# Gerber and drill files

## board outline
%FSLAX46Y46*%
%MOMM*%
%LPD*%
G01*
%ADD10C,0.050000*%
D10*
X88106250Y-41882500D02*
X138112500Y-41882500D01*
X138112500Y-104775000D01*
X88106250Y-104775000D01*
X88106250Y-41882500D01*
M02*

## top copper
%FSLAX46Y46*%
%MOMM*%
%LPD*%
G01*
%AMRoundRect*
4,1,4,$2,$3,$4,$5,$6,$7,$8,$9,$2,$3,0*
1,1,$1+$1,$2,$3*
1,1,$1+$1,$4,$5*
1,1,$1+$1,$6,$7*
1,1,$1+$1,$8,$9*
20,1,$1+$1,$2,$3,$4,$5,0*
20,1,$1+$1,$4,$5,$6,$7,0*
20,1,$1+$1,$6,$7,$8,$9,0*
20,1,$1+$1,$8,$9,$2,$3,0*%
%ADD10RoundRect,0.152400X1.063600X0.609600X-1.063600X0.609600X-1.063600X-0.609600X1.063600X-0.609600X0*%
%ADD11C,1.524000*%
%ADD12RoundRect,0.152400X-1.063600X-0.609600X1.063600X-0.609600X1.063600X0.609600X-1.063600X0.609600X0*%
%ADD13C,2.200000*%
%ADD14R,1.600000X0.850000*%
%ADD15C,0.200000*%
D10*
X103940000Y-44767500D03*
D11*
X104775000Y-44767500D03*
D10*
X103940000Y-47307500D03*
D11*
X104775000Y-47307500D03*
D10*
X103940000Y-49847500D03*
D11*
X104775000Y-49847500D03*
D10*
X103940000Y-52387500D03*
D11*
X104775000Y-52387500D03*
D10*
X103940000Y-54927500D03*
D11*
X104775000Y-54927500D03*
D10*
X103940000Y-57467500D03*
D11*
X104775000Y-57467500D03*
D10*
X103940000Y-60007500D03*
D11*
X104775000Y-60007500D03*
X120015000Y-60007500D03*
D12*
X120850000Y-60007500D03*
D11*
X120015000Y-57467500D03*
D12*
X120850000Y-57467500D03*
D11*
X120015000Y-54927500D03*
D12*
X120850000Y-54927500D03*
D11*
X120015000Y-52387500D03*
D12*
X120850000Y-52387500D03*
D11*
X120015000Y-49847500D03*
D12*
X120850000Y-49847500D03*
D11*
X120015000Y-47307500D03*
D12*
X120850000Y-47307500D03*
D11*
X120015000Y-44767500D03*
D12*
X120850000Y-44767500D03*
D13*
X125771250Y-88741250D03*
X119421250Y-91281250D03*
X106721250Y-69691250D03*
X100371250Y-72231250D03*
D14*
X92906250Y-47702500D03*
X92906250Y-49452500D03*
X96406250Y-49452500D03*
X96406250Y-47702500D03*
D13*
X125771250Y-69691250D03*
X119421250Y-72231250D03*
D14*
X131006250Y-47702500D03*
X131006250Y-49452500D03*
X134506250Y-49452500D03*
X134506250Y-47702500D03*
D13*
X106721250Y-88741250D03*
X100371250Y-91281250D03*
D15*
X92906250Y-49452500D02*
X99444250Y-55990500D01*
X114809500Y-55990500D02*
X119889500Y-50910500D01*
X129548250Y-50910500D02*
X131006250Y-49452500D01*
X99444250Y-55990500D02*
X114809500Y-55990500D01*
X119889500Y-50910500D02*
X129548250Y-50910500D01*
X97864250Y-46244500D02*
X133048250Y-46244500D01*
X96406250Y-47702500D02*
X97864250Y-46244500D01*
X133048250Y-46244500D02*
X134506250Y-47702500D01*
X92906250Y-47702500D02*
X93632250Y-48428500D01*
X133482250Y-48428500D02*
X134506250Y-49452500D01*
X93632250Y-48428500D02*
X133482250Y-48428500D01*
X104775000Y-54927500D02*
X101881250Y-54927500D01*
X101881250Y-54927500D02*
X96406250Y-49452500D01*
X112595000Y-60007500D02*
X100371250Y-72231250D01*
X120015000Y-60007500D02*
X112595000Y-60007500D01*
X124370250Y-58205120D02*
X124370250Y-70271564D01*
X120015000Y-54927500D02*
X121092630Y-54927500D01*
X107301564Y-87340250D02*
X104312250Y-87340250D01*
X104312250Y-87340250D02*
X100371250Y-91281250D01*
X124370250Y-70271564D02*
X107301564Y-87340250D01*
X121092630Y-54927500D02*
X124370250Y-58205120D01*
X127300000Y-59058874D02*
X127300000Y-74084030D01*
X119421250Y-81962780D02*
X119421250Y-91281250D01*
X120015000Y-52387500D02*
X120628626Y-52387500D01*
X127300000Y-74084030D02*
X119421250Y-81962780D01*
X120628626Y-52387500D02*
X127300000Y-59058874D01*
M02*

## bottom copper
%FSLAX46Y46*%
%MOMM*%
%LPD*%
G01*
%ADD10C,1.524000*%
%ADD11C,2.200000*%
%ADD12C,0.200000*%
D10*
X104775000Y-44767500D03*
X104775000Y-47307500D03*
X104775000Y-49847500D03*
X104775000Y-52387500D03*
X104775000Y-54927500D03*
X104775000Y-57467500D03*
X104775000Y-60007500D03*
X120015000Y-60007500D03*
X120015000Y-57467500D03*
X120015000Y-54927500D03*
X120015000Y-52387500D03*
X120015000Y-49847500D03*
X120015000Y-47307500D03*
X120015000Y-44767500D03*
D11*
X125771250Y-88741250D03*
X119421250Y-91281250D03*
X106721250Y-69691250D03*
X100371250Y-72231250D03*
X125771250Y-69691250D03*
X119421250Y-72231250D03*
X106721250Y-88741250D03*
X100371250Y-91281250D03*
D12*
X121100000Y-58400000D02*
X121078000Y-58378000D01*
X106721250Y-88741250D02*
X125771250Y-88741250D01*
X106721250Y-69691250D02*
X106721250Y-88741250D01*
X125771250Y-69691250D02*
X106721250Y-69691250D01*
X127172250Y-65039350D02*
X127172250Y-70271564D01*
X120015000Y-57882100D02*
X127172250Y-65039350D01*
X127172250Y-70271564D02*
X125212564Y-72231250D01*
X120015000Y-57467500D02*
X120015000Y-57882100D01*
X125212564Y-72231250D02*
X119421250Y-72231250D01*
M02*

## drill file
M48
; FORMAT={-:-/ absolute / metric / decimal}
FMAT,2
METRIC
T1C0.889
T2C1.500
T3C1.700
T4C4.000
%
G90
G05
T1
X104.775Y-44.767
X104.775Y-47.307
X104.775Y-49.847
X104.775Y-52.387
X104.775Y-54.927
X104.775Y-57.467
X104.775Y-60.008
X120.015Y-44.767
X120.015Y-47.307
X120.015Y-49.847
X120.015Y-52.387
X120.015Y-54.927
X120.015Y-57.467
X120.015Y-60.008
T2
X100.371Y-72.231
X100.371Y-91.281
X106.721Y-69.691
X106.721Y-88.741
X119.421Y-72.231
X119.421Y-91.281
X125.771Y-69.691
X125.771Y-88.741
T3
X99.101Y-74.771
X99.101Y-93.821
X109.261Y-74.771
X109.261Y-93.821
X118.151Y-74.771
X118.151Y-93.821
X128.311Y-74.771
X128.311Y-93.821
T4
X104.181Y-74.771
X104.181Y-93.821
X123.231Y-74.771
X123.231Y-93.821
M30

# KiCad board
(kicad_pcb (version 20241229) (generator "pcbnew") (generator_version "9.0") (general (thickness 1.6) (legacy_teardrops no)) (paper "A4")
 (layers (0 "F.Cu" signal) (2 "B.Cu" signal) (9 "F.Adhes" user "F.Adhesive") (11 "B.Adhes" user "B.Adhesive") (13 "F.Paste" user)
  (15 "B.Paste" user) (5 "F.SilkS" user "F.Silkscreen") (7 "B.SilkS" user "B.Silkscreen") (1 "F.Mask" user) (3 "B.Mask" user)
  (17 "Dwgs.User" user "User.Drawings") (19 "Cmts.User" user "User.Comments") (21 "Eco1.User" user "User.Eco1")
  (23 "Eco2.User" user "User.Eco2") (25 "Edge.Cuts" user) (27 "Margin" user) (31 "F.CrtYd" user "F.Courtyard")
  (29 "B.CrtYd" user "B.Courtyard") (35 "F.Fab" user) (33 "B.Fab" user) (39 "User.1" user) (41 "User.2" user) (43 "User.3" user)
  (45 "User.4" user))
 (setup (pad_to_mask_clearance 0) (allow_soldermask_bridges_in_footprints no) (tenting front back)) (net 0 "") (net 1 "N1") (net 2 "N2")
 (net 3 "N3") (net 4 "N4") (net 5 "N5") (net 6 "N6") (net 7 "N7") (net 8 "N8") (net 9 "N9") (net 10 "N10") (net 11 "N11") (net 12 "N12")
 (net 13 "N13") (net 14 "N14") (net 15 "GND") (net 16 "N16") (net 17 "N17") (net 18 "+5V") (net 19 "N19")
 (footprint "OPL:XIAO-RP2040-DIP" (layer "F.Cu") (at 112.395 52.3875)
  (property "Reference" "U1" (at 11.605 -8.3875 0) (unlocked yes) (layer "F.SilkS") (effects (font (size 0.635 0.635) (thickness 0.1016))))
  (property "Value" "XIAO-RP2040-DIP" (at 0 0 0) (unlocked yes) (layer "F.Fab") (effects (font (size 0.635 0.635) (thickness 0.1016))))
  (pad "1" smd roundrect (at -8.455 -7.62 180) (size 2.432 1.524) (layers "F.Cu" "F.Mask") (roundrect_rratio 0.1) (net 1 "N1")
   (thermal_bridge_angle 45))
  (pad "1" thru_hole circle (at -7.62 -7.62 180) (size 1.524 1.524) (drill 0.889) (layers "*.Cu" "*.Mask") (remove_unused_layers no)
   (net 1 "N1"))
  (pad "2" smd roundrect (at -8.455 -5.08 180) (size 2.432 1.524) (layers "F.Cu" "F.Mask") (roundrect_rratio 0.1) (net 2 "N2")
   (thermal_bridge_angle 45))
  (pad "2" thru_hole circle (at -7.62 -5.08 180) (size 1.524 1.524) (drill 0.889) (layers "*.Cu" "*.Mask") (remove_unused_layers no)
   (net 2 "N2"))
  (pad "3" smd roundrect (at -8.455 -2.54 180) (size 2.432 1.524) (layers "F.Cu" "F.Mask") (roundrect_rratio 0.1) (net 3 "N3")
   (thermal_bridge_angle 45))
  (pad "3" thru_hole circle (at -7.62 -2.54 180) (size 1.524 1.524) (drill 0.889) (layers "*.Cu" "*.Mask") (remove_unused_layers no)
   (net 3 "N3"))
  (pad "4" smd roundrect (at -8.455 0 180) (size 2.432 1.524) (layers "F.Cu" "F.Mask") (roundrect_rratio 0.1) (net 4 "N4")
   (thermal_bridge_angle 45))
  (pad "4" thru_hole circle (at -7.62 0 180) (size 1.524 1.524) (drill 0.889) (layers "*.Cu" "*.Mask") (remove_unused_layers no)
   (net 4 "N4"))
  (pad "5" smd roundrect (at -8.455 2.54 180) (size 2.432 1.524) (layers "F.Cu" "F.Mask") (roundrect_rratio 0.1) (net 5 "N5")
   (thermal_bridge_angle 45))
  (pad "5" thru_hole circle (at -7.62 2.54 180) (size 1.524 1.524) (drill 0.889) (layers "*.Cu" "*.Mask") (remove_unused_layers no)
   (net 5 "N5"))
  (pad "6" smd roundrect (at -8.455 5.08 180) (size 2.432 1.524) (layers "F.Cu" "F.Mask") (roundrect_rratio 0.1) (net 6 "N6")
   (thermal_bridge_angle 45))
  (pad "6" thru_hole circle (at -7.62 5.08 180) (size 1.524 1.524) (drill 0.889) (layers "*.Cu" "*.Mask") (remove_unused_layers no)
   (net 6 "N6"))
  (pad "7" smd roundrect (at -8.455 7.62 180) (size 2.432 1.524) (layers "F.Cu" "F.Mask") (roundrect_rratio 0.1) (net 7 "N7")
   (thermal_bridge_angle 45))
  (pad "7" thru_hole circle (at -7.62 7.62 180) (size 1.524 1.524) (drill 0.889) (layers "*.Cu" "*.Mask") (remove_unused_layers no)
   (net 7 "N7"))
  (pad "8" thru_hole circle (at 7.62 7.62) (size 1.524 1.524) (drill 0.889) (layers "*.Cu" "*.Mask") (remove_unused_layers no) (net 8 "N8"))
  (pad "8" smd roundrect (at 8.455 7.62) (size 2.432 1.524) (layers "F.Cu" "F.Mask") (roundrect_rratio 0.1) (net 8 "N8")
   (thermal_bridge_angle 45))
  (pad "9" thru_hole circle (at 7.62 5.08) (size 1.524 1.524) (drill 0.889) (layers "*.Cu" "*.Mask") (remove_unused_layers no) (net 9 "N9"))
  (pad "9" smd roundrect (at 8.455 5.08) (size 2.432 1.524) (layers "F.Cu" "F.Mask") (roundrect_rratio 0.1) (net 9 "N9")
   (thermal_bridge_angle 45))
  (pad "10" thru_hole circle (at 7.62 2.54) (size 1.524 1.524) (drill 0.889) (layers "*.Cu" "*.Mask") (remove_unused_layers no)
   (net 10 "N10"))
  (pad "10" smd roundrect (at 8.455 2.54) (size 2.432 1.524) (layers "F.Cu" "F.Mask") (roundrect_rratio 0.1) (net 10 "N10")
   (thermal_bridge_angle 45))
  (pad "11" thru_hole circle (at 7.62 0) (size 1.524 1.524) (drill 0.889) (layers "*.Cu" "*.Mask") (remove_unused_layers no) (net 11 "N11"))
  (pad "11" smd roundrect (at 8.455 0) (size 2.432 1.524) (layers "F.Cu" "F.Mask") (roundrect_rratio 0.1) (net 11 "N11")
   (thermal_bridge_angle 45))
  (pad "12" thru_hole circle (at 7.62 -2.54) (size 1.524 1.524) (drill 0.889) (layers "*.Cu" "*.Mask") (remove_unused_layers no)
   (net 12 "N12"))
  (pad "12" smd roundrect (at 8.455 -2.54) (size 2.432 1.524) (layers "F.Cu" "F.Mask") (roundrect_rratio 0.1) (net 12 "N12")
   (thermal_bridge_angle 45))
  (pad "13" thru_hole circle (at 7.62 -5.08) (size 1.524 1.524) (drill 0.889) (layers "*.Cu" "*.Mask") (remove_unused_layers no)
   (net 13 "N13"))
  (pad "13" smd roundrect (at 8.455 -5.08) (size 2.432 1.524) (layers "F.Cu" "F.Mask") (roundrect_rratio 0.1) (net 13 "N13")
   (thermal_bridge_angle 45))
  (pad "14" thru_hole circle (at 7.62 -7.62) (size 1.524 1.524) (drill 0.889) (layers "*.Cu" "*.Mask") (remove_unused_layers no)
   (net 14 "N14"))
  (pad "14" smd roundrect (at 8.455 -7.62) (size 2.432 1.524) (layers "F.Cu" "F.Mask") (roundrect_rratio 0.1) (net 14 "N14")
   (thermal_bridge_angle 45)))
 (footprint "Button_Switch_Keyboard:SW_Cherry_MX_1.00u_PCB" (layer "F.Cu") (at 125.77125 88.74125)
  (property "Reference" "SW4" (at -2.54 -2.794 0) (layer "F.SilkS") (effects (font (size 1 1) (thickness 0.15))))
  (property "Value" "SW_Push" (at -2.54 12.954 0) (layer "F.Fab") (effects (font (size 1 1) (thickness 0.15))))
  (pad "" np_thru_hole circle (at -7.62 5.08) (size 1.7 1.7) (drill 1.7) (layers "*.Cu" "*.Mask"))
  (pad "" np_thru_hole circle (at -2.54 5.08) (size 4 4) (drill 4) (layers "*.Cu" "*.Mask"))
  (pad "" np_thru_hole circle (at 2.54 5.08) (size 1.7 1.7) (drill 1.7) (layers "*.Cu" "*.Mask"))
  (pad "1" thru_hole circle (at 0 0) (size 2.2 2.2) (drill 1.5) (layers "*.Cu" "*.Mask") (remove_unused_layers no) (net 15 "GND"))
  (pad "2" thru_hole circle (at -6.35 2.54) (size 2.2 2.2) (drill 1.5) (layers "*.Cu" "*.Mask") (remove_unused_layers no) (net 11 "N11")))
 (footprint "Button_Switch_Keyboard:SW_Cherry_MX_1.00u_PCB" (layer "F.Cu") (at 106.72125 69.69125)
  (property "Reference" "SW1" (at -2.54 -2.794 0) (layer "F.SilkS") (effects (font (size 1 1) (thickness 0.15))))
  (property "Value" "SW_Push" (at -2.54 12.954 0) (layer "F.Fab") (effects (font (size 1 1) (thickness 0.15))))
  (pad "" np_thru_hole circle (at -7.62 5.08) (size 1.7 1.7) (drill 1.7) (layers "*.Cu" "*.Mask"))
  (pad "" np_thru_hole circle (at -2.54 5.08) (size 4 4) (drill 4) (layers "*.Cu" "*.Mask"))
  (pad "" np_thru_hole circle (at 2.54 5.08) (size 1.7 1.7) (drill 1.7) (layers "*.Cu" "*.Mask"))
  (pad "1" thru_hole circle (at 0 0) (size 2.2 2.2) (drill 1.5) (layers "*.Cu" "*.Mask") (remove_unused_layers no) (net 15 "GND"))
  (pad "2" thru_hole circle (at -6.35 2.54) (size 2.2 2.2) (drill 1.5) (layers "*.Cu" "*.Mask") (remove_unused_layers no) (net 8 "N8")))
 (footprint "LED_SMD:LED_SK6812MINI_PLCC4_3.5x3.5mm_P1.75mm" (layer "F.Cu") (at 94.65625 48.5775)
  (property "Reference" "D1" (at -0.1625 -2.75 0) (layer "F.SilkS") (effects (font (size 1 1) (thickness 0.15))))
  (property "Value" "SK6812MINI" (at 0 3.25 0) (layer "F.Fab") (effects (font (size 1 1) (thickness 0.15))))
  (pad "1" smd rect (at -1.75 -0.875) (size 1.6 0.85) (layers "F.Cu" "F.Mask" "F.Paste") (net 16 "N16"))
  (pad "2" smd rect (at -1.75 0.875) (size 1.6 0.85) (layers "F.Cu" "F.Mask" "F.Paste") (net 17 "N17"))
  (pad "3" smd rect (at 1.75 0.875) (size 1.6 0.85) (layers "F.Cu" "F.Mask" "F.Paste") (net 5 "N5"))
  (pad "4" smd rect (at 1.75 -0.875) (size 1.6 0.85) (layers "F.Cu" "F.Mask" "F.Paste") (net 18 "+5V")))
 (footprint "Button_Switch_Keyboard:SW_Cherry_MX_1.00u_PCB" (layer "F.Cu") (at 125.77125 69.69125)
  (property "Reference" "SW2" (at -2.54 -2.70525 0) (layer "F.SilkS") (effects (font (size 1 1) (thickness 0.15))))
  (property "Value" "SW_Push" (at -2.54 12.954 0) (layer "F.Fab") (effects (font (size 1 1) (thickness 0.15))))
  (pad "" np_thru_hole circle (at -7.62 5.08) (size 1.7 1.7) (drill 1.7) (layers "*.Cu" "*.Mask"))
  (pad "" np_thru_hole circle (at -2.54 5.08) (size 4 4) (drill 4) (layers "*.Cu" "*.Mask"))
  (pad "" np_thru_hole circle (at 2.54 5.08) (size 1.7 1.7) (drill 1.7) (layers "*.Cu" "*.Mask"))
  (pad "1" thru_hole circle (at 0 0) (size 2.2 2.2) (drill 1.5) (layers "*.Cu" "*.Mask") (remove_unused_layers no) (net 15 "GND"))
  (pad "2" thru_hole circle (at -6.35 2.54) (size 2.2 2.2) (drill 1.5) (layers "*.Cu" "*.Mask") (remove_unused_layers no) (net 9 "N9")))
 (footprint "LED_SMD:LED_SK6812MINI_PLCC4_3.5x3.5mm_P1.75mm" (layer "F.Cu") (at 132.75625 48.5775)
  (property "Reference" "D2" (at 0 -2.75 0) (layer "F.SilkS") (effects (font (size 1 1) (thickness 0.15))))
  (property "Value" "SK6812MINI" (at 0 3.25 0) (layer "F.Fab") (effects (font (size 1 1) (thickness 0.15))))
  (pad "1" smd rect (at -1.75 -0.875) (size 1.6 0.85) (layers "F.Cu" "F.Mask" "F.Paste") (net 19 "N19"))
  (pad "2" smd rect (at -1.75 0.875) (size 1.6 0.85) (layers "F.Cu" "F.Mask" "F.Paste") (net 17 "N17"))
  (pad "3" smd rect (at 1.75 0.875) (size 1.6 0.85) (layers "F.Cu" "F.Mask" "F.Paste") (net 16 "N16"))
  (pad "4" smd rect (at 1.75 -0.875) (size 1.6 0.85) (layers "F.Cu" "F.Mask" "F.Paste") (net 18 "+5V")))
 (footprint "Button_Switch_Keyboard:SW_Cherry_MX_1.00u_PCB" (layer "F.Cu") (at 106.72125 88.74125)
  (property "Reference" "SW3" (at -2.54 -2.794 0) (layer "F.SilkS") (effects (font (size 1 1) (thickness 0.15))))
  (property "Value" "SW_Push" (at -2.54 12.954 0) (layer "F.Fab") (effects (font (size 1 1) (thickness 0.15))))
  (pad "" np_thru_hole circle (at -7.62 5.08) (size 1.7 1.7) (drill 1.7) (layers "*.Cu" "*.Mask"))
  (pad "" np_thru_hole circle (at -2.54 5.08) (size 4 4) (drill 4) (layers "*.Cu" "*.Mask"))
  (pad "" np_thru_hole circle (at 2.54 5.08) (size 1.7 1.7) (drill 1.7) (layers "*.Cu" "*.Mask"))
  (pad "1" thru_hole circle (at 0 0) (size 2.2 2.2) (drill 1.5) (layers "*.Cu" "*.Mask") (remove_unused_layers no) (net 15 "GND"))
  (pad "2" thru_hole circle (at -6.35 2.54) (size 2.2 2.2) (drill 1.5) (layers "*.Cu" "*.Mask") (remove_unused_layers no) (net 10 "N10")))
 (gr_rect (start 88.10625 41.8825) (end 138.1125 104.775) (stroke (width 0.05) (type default)) (fill no) (layer "Edge.Cuts"))
 (segment (start 121.1 58.4) (end 121.078 58.378) (width 0.2) (layer "B.Cu") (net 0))
 (segment (start 92.90625 49.4525) (end 99.44425 55.9905) (width 0.2) (layer "F.Cu") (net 17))
 (segment (start 114.8095 55.9905) (end 119.8895 50.9105) (width 0.2) (layer "F.Cu") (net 17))
 (segment (start 129.54825 50.9105) (end 131.00625 49.4525) (width 0.2) (layer "F.Cu") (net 17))
 (segment (start 99.44425 55.9905) (end 114.8095 55.9905) (width 0.2) (layer "F.Cu") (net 17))
 (segment (start 119.8895 50.9105) (end 129.54825 50.9105) (width 0.2) (layer "F.Cu") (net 17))
 (segment (start 97.86425 46.2445) (end 133.04825 46.2445) (width 0.2) (layer "F.Cu") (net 18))
 (segment (start 96.40625 47.7025) (end 97.86425 46.2445) (width 0.2) (layer "F.Cu") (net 18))
 (segment (start 133.04825 46.2445) (end 134.50625 47.7025) (width 0.2) (layer "F.Cu") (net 18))
 (segment (start 92.90625 47.7025) (end 93.63225 48.4285) (width 0.2) (layer "F.Cu") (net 16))
 (segment (start 133.48225 48.4285) (end 134.50625 49.4525) (width 0.2) (layer "F.Cu") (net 16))
 (segment (start 93.63225 48.4285) (end 133.48225 48.4285) (width 0.2) (layer "F.Cu") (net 16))
 (segment (start 104.775 54.9275) (end 101.88125 54.9275) (width 0.2) (layer "F.Cu") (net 5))
 (segment (start 101.88125 54.9275) (end 96.40625 49.4525) (width 0.2) (layer "F.Cu") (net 5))
 (segment (start 106.72125 88.74125) (end 125.77125 88.74125) (width 0.2) (layer "B.Cu") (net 15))
 (segment (start 106.72125 69.69125) (end 106.72125 88.74125) (width 0.2) (layer "B.Cu") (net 15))
 (segment (start 125.77125 69.69125) (end 106.72125 69.69125) (width 0.2) (layer "B.Cu") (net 15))
 (segment (start 112.595 60.0075) (end 100.37125 72.23125) (width 0.2) (layer "F.Cu") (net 8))
 (segment (start 120.015 60.0075) (end 112.595 60.0075) (width 0.2) (layer "F.Cu") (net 8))
 (segment (start 127.17225 65.03935) (end 127.17225 70.271564) (width 0.2) (layer "B.Cu") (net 9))
 (segment (start 120.015 57.8821) (end 127.17225 65.03935) (width 0.2) (layer "B.Cu") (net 9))
 (segment (start 127.17225 70.271564) (end 125.212564 72.23125) (width 0.2) (layer "B.Cu") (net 9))
 (segment (start 120.015 57.4675) (end 120.015 57.8821) (width 0.2) (layer "B.Cu") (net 9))
 (segment (start 125.212564 72.23125) (end 119.42125 72.23125) (width 0.2) (layer "B.Cu") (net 9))
 (segment (start 124.37025 58.20512) (end 124.37025 70.271564) (width 0.2) (layer "F.Cu") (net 10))
 (segment (start 120.015 54.9275) (end 121.09263 54.9275) (width 0.2) (layer "F.Cu") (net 10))
 (segment (start 107.301564 87.34025) (end 104.31225 87.34025) (width 0.2) (layer "F.Cu") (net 10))
 (segment (start 104.31225 87.34025) (end 100.37125 91.28125) (width 0.2) (layer "F.Cu") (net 10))
 (segment (start 124.37025 70.271564) (end 107.301564 87.34025) (width 0.2) (layer "F.Cu") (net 10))
 (segment (start 121.09263 54.9275) (end 124.37025 58.20512) (width 0.2) (layer "F.Cu") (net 10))
 (segment (start 127.3 59.058874) (end 127.3 74.08403) (width 0.2) (layer "F.Cu") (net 11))
 (segment (start 119.42125 81.96278) (end 119.42125 91.28125) (width 0.2) (layer "F.Cu") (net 11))
 (segment (start 120.015 52.3875) (end 120.628626 52.3875) (width 0.2) (layer "F.Cu") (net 11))
 (segment (start 127.3 74.08403) (end 119.42125 81.96278) (width 0.2) (layer "F.Cu") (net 11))
 (segment (start 120.628626 52.3875) (end 127.3 59.058874) (width 0.2) (layer "F.Cu") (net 11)))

